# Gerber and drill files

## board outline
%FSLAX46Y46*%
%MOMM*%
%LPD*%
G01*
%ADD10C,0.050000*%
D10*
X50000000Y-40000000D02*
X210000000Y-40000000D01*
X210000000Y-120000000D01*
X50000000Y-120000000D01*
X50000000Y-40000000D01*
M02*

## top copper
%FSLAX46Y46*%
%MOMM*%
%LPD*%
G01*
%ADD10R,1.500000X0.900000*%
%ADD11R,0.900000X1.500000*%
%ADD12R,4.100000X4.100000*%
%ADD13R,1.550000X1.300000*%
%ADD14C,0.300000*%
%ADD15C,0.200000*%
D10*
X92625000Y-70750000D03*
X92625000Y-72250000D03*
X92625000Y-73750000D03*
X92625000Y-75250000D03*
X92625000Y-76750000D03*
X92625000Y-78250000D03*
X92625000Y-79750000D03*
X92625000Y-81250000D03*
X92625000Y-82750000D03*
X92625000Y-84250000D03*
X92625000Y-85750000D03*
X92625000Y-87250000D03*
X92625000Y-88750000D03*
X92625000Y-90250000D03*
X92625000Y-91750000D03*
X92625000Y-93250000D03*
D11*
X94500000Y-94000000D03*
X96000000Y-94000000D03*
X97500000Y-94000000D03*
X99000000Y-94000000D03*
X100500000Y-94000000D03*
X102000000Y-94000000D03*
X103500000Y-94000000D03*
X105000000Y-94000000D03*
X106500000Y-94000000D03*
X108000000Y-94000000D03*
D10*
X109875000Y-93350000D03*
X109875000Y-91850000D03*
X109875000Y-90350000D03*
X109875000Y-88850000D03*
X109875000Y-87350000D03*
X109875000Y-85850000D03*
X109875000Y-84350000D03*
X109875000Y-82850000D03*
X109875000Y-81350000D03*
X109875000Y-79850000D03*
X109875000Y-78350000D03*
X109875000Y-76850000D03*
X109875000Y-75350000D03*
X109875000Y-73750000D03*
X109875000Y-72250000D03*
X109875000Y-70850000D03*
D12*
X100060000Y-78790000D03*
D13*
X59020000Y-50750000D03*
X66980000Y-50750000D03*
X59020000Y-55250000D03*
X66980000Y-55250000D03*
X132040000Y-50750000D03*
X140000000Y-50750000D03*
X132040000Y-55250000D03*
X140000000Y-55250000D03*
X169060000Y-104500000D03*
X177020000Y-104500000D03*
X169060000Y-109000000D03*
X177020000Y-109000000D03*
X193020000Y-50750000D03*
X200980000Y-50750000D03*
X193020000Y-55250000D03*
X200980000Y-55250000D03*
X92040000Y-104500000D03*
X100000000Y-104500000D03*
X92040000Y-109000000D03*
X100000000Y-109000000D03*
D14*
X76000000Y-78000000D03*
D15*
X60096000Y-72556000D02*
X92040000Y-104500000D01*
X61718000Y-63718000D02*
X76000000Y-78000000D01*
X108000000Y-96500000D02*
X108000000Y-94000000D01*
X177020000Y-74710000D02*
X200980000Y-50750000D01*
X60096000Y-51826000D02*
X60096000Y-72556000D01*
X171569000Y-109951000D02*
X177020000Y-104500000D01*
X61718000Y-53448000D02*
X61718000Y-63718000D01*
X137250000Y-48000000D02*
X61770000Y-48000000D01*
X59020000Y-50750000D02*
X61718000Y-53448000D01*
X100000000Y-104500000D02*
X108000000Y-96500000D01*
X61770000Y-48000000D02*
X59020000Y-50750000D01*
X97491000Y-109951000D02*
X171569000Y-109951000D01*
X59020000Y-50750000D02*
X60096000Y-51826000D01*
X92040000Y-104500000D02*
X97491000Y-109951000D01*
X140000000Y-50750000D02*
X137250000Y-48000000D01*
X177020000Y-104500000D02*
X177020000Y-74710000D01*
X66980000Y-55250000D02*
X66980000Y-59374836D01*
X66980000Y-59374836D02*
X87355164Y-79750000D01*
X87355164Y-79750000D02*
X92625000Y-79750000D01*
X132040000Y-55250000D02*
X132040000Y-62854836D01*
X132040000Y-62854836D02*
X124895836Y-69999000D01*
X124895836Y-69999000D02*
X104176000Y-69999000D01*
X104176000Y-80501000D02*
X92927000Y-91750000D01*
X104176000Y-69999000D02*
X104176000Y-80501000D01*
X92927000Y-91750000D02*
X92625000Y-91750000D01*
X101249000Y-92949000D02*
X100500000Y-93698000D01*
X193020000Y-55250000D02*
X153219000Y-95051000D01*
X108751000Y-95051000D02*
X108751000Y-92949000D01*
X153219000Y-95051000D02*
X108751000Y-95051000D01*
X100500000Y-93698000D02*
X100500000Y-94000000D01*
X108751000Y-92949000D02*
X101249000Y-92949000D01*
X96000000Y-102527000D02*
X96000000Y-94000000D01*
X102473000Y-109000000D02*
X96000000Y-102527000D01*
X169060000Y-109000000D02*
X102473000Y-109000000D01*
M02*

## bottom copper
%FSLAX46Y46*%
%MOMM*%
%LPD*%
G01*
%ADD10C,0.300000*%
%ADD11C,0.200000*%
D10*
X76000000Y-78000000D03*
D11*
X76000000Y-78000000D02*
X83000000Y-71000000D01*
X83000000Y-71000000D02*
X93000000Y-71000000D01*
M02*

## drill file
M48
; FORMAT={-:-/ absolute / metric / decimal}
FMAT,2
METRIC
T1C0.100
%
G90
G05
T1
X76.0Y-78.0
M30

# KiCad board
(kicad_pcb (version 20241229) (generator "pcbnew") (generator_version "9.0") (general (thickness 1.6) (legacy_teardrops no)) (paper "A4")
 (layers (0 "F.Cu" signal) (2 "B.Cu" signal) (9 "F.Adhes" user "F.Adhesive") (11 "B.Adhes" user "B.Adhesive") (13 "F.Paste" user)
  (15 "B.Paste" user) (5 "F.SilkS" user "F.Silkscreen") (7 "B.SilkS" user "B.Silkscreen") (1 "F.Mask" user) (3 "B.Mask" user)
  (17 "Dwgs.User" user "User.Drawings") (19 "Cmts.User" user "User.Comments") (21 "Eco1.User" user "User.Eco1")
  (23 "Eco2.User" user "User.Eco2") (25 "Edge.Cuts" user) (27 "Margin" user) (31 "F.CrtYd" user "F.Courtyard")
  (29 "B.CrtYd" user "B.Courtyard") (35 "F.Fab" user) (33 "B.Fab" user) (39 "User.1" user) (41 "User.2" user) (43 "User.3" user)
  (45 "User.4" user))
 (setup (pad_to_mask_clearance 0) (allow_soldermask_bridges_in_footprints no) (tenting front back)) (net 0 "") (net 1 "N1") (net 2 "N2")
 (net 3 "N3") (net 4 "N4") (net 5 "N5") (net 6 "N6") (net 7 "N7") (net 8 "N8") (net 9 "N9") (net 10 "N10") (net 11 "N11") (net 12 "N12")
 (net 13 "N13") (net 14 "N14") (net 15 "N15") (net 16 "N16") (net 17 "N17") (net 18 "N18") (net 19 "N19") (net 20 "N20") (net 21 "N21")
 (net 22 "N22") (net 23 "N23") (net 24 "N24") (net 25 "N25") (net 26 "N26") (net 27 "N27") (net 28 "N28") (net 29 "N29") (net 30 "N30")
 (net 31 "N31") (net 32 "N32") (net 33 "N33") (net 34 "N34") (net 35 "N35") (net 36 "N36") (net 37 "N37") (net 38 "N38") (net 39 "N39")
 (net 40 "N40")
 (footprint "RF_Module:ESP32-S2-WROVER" (layer "F.Cu") (at 101.25 82.525)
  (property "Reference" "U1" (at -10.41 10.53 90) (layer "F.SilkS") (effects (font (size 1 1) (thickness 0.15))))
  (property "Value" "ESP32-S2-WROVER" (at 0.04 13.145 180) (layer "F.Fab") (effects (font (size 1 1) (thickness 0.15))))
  (pad "" smd roundrect (at -2.52 -5.065) (size 1.07 1.07) (layers "F.Paste") (roundrect_rratio 0.233645))
  (pad "" smd roundrect (at -2.52 -3.735) (size 1.07 1.07) (layers "F.Paste") (roundrect_rratio 0.233645))
  (pad "" smd roundrect (at -2.52 -2.405) (size 1.07 1.07) (layers "F.Paste") (roundrect_rratio 0.233645))
  (pad "" smd roundrect (at -1.19 -5.065) (size 1.07 1.07) (layers "F.Paste") (roundrect_rratio 0.233645))
  (pad "" smd roundrect (at -1.19 -3.735) (size 1.07 1.07) (layers "F.Paste") (roundrect_rratio 0.233645))
  (pad "" smd roundrect (at -1.19 -2.405) (size 1.07 1.07) (layers "F.Paste") (roundrect_rratio 0.233645))
  (pad "" smd roundrect (at 0.14 -5.065) (size 1.07 1.07) (layers "F.Paste") (roundrect_rratio 0.233645))
  (pad "" smd roundrect (at 0.14 -3.735) (size 1.07 1.07) (layers "F.Paste") (roundrect_rratio 0.233645))
  (pad "" smd roundrect (at 0.14 -2.405) (size 1.07 1.07) (layers "F.Paste") (roundrect_rratio 0.233645))
  (pad "1" smd rect (at -8.625 -11.775) (size 1.5 0.9) (layers "F.Cu" "F.Mask" "F.Paste") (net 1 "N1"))
  (pad "2" smd rect (at -8.625 -10.275) (size 1.5 0.9) (layers "F.Cu" "F.Mask" "F.Paste") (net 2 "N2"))
  (pad "3" smd rect (at -8.625 -8.775) (size 1.5 0.9) (layers "F.Cu" "F.Mask" "F.Paste") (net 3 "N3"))
  (pad "4" smd rect (at -8.625 -7.275) (size 1.5 0.9) (layers "F.Cu" "F.Mask" "F.Paste") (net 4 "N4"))
  (pad "5" smd rect (at -8.625 -5.775) (size 1.5 0.9) (layers "F.Cu" "F.Mask" "F.Paste") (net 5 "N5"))
  (pad "6" smd rect (at -8.625 -4.275) (size 1.5 0.9) (layers "F.Cu" "F.Mask" "F.Paste") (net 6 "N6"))
  (pad "7" smd rect (at -8.625 -2.775) (size 1.5 0.9) (layers "F.Cu" "F.Mask" "F.Paste") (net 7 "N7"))
  (pad "8" smd rect (at -8.625 -1.275) (size 1.5 0.9) (layers "F.Cu" "F.Mask" "F.Paste") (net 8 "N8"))
  (pad "9" smd rect (at -8.625 0.225) (size 1.5 0.9) (layers "F.Cu" "F.Mask" "F.Paste") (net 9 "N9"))
  (pad "10" smd rect (at -8.625 1.725) (size 1.5 0.9) (layers "F.Cu" "F.Mask" "F.Paste") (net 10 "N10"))
  (pad "11" smd rect (at -8.625 3.225) (size 1.5 0.9) (layers "F.Cu" "F.Mask" "F.Paste") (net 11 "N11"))
  (pad "12" smd rect (at -8.625 4.725) (size 1.5 0.9) (layers "F.Cu" "F.Mask" "F.Paste") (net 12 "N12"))
  (pad "13" smd rect (at -8.625 6.225) (size 1.5 0.9) (layers "F.Cu" "F.Mask" "F.Paste") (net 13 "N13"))
  (pad "14" smd rect (at -8.625 7.725) (size 1.5 0.9) (layers "F.Cu" "F.Mask" "F.Paste") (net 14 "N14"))
  (pad "15" smd rect (at -8.625 9.225 180) (size 1.5 0.9) (layers "F.Cu" "F.Mask" "F.Paste") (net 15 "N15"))
  (pad "16" smd rect (at -8.625 10.725 180) (size 1.5 0.9) (layers "F.Cu" "F.Mask" "F.Paste") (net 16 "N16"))
  (pad "17" smd rect (at -6.75 11.475) (size 0.9 1.5) (layers "F.Cu" "F.Mask" "F.Paste") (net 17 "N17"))
  (pad "18" smd rect (at -5.25 11.475) (size 0.9 1.5) (layers "F.Cu" "F.Mask" "F.Paste") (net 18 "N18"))
  (pad "19" smd rect (at -3.75 11.475) (size 0.9 1.5) (layers "F.Cu" "F.Mask" "F.Paste") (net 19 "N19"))
  (pad "20" smd rect (at -2.25 11.475) (size 0.9 1.5) (layers "F.Cu" "F.Mask" "F.Paste") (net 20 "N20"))
  (pad "21" smd rect (at -0.75 11.475) (size 0.9 1.5) (layers "F.Cu" "F.Mask" "F.Paste") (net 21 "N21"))
  (pad "22" smd rect (at 0.75 11.475) (size 0.9 1.5) (layers "F.Cu" "F.Mask" "F.Paste") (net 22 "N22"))
  (pad "23" smd rect (at 2.25 11.475) (size 0.9 1.5) (layers "F.Cu" "F.Mask" "F.Paste") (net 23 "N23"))
  (pad "24" smd rect (at 3.75 11.475) (size 0.9 1.5) (layers "F.Cu" "F.Mask" "F.Paste") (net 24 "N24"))
  (pad "25" smd rect (at 5.25 11.475) (size 0.9 1.5) (layers "F.Cu" "F.Mask" "F.Paste") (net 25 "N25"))
  (pad "26" smd rect (at 6.75 11.475) (size 0.9 1.5) (layers "F.Cu" "F.Mask" "F.Paste") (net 1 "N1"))
  (pad "27" smd rect (at 8.625 10.825) (size 1.5 0.9) (layers "F.Cu" "F.Mask" "F.Paste") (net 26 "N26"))
  (pad "28" smd rect (at 8.625 9.325) (size 1.5 0.9) (layers "F.Cu" "F.Mask" "F.Paste") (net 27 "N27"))
  (pad "29" smd rect (at 8.625 7.825) (size 1.5 0.9) (layers "F.Cu" "F.Mask" "F.Paste") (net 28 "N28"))
  (pad "30" smd rect (at 8.625 6.325) (size 1.5 0.9) (layers "F.Cu" "F.Mask" "F.Paste") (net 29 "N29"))
  (pad "31" smd rect (at 8.625 4.825) (size 1.5 0.9) (layers "F.Cu" "F.Mask" "F.Paste") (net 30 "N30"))
  (pad "32" smd rect (at 8.625 3.325) (size 1.5 0.9) (layers "F.Cu" "F.Mask" "F.Paste") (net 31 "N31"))
  (pad "33" smd rect (at 8.625 1.825) (size 1.5 0.9) (layers "F.Cu" "F.Mask" "F.Paste") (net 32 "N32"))
  (pad "34" smd rect (at 8.625 0.325) (size 1.5 0.9) (layers "F.Cu" "F.Mask" "F.Paste") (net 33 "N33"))
  (pad "35" smd rect (at 8.625 -1.175) (size 1.5 0.9) (layers "F.Cu" "F.Mask" "F.Paste") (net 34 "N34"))
  (pad "36" smd rect (at 8.625 -2.675) (size 1.5 0.9) (layers "F.Cu" "F.Mask" "F.Paste") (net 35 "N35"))
  (pad "37" smd rect (at 8.625 -4.175) (size 1.5 0.9) (layers "F.Cu" "F.Mask" "F.Paste") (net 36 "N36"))
  (pad "38" smd rect (at 8.625 -5.675) (size 1.5 0.9) (layers "F.Cu" "F.Mask" "F.Paste") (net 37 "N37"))
  (pad "39" smd rect (at 8.625 -7.175) (size 1.5 0.9) (layers "F.Cu" "F.Mask" "F.Paste") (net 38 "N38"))
  (pad "40" smd rect (at 8.625 -8.775) (size 1.5 0.9) (layers "F.Cu" "F.Mask" "F.Paste") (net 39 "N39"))
  (pad "41" smd rect (at 8.625 -10.275) (size 1.5 0.9) (layers "F.Cu" "F.Mask" "F.Paste") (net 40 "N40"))
  (pad "42" smd rect (at 8.625 -11.675) (size 1.5 0.9) (layers "F.Cu" "F.Mask" "F.Paste") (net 1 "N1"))
  (pad "43" smd rect (at -1.19 -3.735) (size 4.1 4.1) (layers "F.Cu" "F.Mask") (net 1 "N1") (zone_connect 2))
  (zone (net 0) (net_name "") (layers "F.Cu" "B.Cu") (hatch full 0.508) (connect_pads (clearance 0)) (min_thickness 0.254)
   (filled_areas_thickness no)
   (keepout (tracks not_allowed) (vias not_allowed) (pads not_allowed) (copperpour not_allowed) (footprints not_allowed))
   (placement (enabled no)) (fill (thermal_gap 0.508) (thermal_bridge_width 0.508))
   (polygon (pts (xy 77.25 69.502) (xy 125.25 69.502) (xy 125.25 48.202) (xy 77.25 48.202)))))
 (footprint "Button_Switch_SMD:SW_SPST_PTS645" (layer "F.Cu") (at 63 53)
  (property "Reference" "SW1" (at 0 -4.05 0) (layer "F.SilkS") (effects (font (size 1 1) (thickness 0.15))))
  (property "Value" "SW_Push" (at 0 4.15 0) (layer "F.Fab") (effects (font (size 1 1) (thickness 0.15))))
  (pad "1" smd rect (at -3.98 -2.25) (size 1.55 1.3) (layers "F.Cu" "F.Mask" "F.Paste") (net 1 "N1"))
  (pad "1" smd rect (at 3.98 -2.25) (size 1.55 1.3) (layers "F.Cu" "F.Mask" "F.Paste") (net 1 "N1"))
  (pad "2" smd rect (at -3.98 2.25) (size 1.55 1.3) (layers "F.Cu" "F.Mask" "F.Paste") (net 7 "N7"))
  (pad "2" smd rect (at 3.98 2.25) (size 1.55 1.3) (layers "F.Cu" "F.Mask" "F.Paste") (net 7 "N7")))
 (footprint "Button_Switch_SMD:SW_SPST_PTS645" (layer "F.Cu") (at 136.02 53)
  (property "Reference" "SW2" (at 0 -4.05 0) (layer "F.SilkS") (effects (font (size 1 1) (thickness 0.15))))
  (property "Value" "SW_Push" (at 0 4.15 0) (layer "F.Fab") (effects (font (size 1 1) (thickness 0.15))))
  (pad "1" smd rect (at -3.98 -2.25) (size 1.55 1.3) (layers "F.Cu" "F.Mask" "F.Paste") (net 1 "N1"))
  (pad "1" smd rect (at 3.98 -2.25) (size 1.55 1.3) (layers "F.Cu" "F.Mask" "F.Paste") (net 1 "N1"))
  (pad "2" smd rect (at -3.98 2.25) (size 1.55 1.3) (layers "F.Cu" "F.Mask" "F.Paste") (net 15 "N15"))
  (pad "2" smd rect (at 3.98 2.25) (size 1.55 1.3) (layers "F.Cu" "F.Mask" "F.Paste") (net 15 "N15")))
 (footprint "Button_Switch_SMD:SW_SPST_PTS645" (layer "F.Cu") (at 173.04 106.75)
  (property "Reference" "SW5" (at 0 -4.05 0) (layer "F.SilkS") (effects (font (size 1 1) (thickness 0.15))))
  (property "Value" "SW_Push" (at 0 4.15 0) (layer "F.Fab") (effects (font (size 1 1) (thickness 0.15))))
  (pad "1" smd rect (at -3.98 -2.25) (size 1.55 1.3) (layers "F.Cu" "F.Mask" "F.Paste") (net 1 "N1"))
  (pad "1" smd rect (at 3.98 -2.25) (size 1.55 1.3) (layers "F.Cu" "F.Mask" "F.Paste") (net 1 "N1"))
  (pad "2" smd rect (at -3.98 2.25) (size 1.55 1.3) (layers "F.Cu" "F.Mask" "F.Paste") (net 18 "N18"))
  (pad "2" smd rect (at 3.98 2.25) (size 1.55 1.3) (layers "F.Cu" "F.Mask" "F.Paste") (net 18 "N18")))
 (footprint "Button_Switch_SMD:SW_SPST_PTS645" (layer "F.Cu") (at 197 53)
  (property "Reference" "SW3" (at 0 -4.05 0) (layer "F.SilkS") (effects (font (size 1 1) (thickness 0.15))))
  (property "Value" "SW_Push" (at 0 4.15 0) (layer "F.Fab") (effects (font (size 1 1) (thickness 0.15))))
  (pad "1" smd rect (at -3.98 -2.25) (size 1.55 1.3) (layers "F.Cu" "F.Mask" "F.Paste") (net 1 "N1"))
  (pad "1" smd rect (at 3.98 -2.25) (size 1.55 1.3) (layers "F.Cu" "F.Mask" "F.Paste") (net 1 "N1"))
  (pad "2" smd rect (at -3.98 2.25) (size 1.55 1.3) (layers "F.Cu" "F.Mask" "F.Paste") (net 21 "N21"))
  (pad "2" smd rect (at 3.98 2.25) (size 1.55 1.3) (layers "F.Cu" "F.Mask" "F.Paste") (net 21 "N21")))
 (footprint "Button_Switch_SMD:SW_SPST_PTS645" (layer "F.Cu") (at 96.02 106.75)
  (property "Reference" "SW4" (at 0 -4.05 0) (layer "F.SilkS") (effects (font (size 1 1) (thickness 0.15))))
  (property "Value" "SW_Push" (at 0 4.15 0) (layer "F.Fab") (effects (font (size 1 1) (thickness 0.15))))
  (pad "1" smd rect (at -3.98 -2.25) (size 1.55 1.3) (layers "F.Cu" "F.Mask" "F.Paste") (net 1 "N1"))
  (pad "1" smd rect (at 3.98 -2.25) (size 1.55 1.3) (layers "F.Cu" "F.Mask" "F.Paste") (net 1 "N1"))
  (pad "2" smd rect (at -3.98 2.25) (size 1.55 1.3) (layers "F.Cu" "F.Mask" "F.Paste") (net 11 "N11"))
  (pad "2" smd rect (at 3.98 2.25) (size 1.55 1.3) (layers "F.Cu" "F.Mask" "F.Paste") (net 11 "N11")))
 (gr_rect (start 50 40) (end 210 120) (stroke (width 0.05) (type solid)) (fill no) (layer "Edge.Cuts"))
 (segment (start 60.096 72.556) (end 92.04 104.5) (width 0.2) (layer "F.Cu") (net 1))
 (segment (start 61.718 63.718) (end 76 78) (width 0.2) (layer "F.Cu") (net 1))
 (segment (start 108 96.5) (end 108 94) (width 0.2) (layer "F.Cu") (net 1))
 (segment (start 177.02 74.71) (end 200.98 50.75) (width 0.2) (layer "F.Cu") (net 1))
 (segment (start 60.096 51.826) (end 60.096 72.556) (width 0.2) (layer "F.Cu") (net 1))
 (segment (start 171.569 109.951) (end 177.02 104.5) (width 0.2) (layer "F.Cu") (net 1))
 (segment (start 61.718 53.448) (end 61.718 63.718) (width 0.2) (layer "F.Cu") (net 1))
 (segment (start 137.25 48) (end 61.77 48) (width 0.2) (layer "F.Cu") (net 1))
 (segment (start 59.02 50.75) (end 61.718 53.448) (width 0.2) (layer "F.Cu") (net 1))
 (segment (start 100 104.5) (end 108 96.5) (width 0.2) (layer "F.Cu") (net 1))
 (segment (start 61.77 48) (end 59.02 50.75) (width 0.2) (layer "F.Cu") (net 1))
 (segment (start 97.491 109.951) (end 171.569 109.951) (width 0.2) (layer "F.Cu") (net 1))
 (segment (start 59.02 50.75) (end 60.096 51.826) (width 0.2) (layer "F.Cu") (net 1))
 (segment (start 92.04 104.5) (end 97.491 109.951) (width 0.2) (layer "F.Cu") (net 1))
 (segment (start 140 50.75) (end 137.25 48) (width 0.2) (layer "F.Cu") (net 1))
 (segment (start 177.02 104.5) (end 177.02 74.71) (width 0.2) (layer "F.Cu") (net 1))
 (via micro (at 76 78) (size 0.3) (drill 0.1) (layers "F.Cu" "B.Cu") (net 1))
 (segment (start 76 78) (end 83 71) (width 0.2) (layer "B.Cu") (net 1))
 (segment (start 83 71) (end 93 71) (width 0.2) (layer "B.Cu") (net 1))
 (segment (start 66.98 55.25) (end 66.98 59.374836) (width 0.2) (layer "F.Cu") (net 7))
 (segment (start 66.98 59.374836) (end 87.355164 79.75) (width 0.2) (layer "F.Cu") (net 7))
 (segment (start 87.355164 79.75) (end 92.625 79.75) (width 0.2) (layer "F.Cu") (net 7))
 (segment (start 132.04 55.25) (end 132.04 62.854836) (width 0.2) (layer "F.Cu") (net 15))
 (segment (start 132.04 62.854836) (end 124.895836 69.999) (width 0.2) (layer "F.Cu") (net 15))
 (segment (start 124.895836 69.999) (end 104.176 69.999) (width 0.2) (layer "F.Cu") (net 15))
 (segment (start 104.176 80.501) (end 92.927 91.75) (width 0.2) (layer "F.Cu") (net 15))
 (segment (start 104.176 69.999) (end 104.176 80.501) (width 0.2) (layer "F.Cu") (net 15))
 (segment (start 92.927 91.75) (end 92.625 91.75) (width 0.2) (layer "F.Cu") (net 15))
 (segment (start 101.249 92.949) (end 100.5 93.698) (width 0.2) (layer "F.Cu") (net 21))
 (segment (start 193.02 55.25) (end 153.219 95.051) (width 0.2) (layer "F.Cu") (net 21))
 (segment (start 108.751 95.051) (end 108.751 92.949) (width 0.2) (layer "F.Cu") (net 21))
 (segment (start 153.219 95.051) (end 108.751 95.051) (width 0.2) (layer "F.Cu") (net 21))
 (segment (start 100.5 93.698) (end 100.5 94) (width 0.2) (layer "F.Cu") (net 21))
 (segment (start 108.751 92.949) (end 101.249 92.949) (width 0.2) (layer "F.Cu") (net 21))
 (segment (start 96 102.527) (end 96 94) (width 0.2) (layer "F.Cu") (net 18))
 (segment (start 102.473 109) (end 96 102.527) (width 0.2) (layer "F.Cu") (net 18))
 (segment (start 169.06 109) (end 102.473 109) (width 0.2) (layer "F.Cu") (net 18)))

